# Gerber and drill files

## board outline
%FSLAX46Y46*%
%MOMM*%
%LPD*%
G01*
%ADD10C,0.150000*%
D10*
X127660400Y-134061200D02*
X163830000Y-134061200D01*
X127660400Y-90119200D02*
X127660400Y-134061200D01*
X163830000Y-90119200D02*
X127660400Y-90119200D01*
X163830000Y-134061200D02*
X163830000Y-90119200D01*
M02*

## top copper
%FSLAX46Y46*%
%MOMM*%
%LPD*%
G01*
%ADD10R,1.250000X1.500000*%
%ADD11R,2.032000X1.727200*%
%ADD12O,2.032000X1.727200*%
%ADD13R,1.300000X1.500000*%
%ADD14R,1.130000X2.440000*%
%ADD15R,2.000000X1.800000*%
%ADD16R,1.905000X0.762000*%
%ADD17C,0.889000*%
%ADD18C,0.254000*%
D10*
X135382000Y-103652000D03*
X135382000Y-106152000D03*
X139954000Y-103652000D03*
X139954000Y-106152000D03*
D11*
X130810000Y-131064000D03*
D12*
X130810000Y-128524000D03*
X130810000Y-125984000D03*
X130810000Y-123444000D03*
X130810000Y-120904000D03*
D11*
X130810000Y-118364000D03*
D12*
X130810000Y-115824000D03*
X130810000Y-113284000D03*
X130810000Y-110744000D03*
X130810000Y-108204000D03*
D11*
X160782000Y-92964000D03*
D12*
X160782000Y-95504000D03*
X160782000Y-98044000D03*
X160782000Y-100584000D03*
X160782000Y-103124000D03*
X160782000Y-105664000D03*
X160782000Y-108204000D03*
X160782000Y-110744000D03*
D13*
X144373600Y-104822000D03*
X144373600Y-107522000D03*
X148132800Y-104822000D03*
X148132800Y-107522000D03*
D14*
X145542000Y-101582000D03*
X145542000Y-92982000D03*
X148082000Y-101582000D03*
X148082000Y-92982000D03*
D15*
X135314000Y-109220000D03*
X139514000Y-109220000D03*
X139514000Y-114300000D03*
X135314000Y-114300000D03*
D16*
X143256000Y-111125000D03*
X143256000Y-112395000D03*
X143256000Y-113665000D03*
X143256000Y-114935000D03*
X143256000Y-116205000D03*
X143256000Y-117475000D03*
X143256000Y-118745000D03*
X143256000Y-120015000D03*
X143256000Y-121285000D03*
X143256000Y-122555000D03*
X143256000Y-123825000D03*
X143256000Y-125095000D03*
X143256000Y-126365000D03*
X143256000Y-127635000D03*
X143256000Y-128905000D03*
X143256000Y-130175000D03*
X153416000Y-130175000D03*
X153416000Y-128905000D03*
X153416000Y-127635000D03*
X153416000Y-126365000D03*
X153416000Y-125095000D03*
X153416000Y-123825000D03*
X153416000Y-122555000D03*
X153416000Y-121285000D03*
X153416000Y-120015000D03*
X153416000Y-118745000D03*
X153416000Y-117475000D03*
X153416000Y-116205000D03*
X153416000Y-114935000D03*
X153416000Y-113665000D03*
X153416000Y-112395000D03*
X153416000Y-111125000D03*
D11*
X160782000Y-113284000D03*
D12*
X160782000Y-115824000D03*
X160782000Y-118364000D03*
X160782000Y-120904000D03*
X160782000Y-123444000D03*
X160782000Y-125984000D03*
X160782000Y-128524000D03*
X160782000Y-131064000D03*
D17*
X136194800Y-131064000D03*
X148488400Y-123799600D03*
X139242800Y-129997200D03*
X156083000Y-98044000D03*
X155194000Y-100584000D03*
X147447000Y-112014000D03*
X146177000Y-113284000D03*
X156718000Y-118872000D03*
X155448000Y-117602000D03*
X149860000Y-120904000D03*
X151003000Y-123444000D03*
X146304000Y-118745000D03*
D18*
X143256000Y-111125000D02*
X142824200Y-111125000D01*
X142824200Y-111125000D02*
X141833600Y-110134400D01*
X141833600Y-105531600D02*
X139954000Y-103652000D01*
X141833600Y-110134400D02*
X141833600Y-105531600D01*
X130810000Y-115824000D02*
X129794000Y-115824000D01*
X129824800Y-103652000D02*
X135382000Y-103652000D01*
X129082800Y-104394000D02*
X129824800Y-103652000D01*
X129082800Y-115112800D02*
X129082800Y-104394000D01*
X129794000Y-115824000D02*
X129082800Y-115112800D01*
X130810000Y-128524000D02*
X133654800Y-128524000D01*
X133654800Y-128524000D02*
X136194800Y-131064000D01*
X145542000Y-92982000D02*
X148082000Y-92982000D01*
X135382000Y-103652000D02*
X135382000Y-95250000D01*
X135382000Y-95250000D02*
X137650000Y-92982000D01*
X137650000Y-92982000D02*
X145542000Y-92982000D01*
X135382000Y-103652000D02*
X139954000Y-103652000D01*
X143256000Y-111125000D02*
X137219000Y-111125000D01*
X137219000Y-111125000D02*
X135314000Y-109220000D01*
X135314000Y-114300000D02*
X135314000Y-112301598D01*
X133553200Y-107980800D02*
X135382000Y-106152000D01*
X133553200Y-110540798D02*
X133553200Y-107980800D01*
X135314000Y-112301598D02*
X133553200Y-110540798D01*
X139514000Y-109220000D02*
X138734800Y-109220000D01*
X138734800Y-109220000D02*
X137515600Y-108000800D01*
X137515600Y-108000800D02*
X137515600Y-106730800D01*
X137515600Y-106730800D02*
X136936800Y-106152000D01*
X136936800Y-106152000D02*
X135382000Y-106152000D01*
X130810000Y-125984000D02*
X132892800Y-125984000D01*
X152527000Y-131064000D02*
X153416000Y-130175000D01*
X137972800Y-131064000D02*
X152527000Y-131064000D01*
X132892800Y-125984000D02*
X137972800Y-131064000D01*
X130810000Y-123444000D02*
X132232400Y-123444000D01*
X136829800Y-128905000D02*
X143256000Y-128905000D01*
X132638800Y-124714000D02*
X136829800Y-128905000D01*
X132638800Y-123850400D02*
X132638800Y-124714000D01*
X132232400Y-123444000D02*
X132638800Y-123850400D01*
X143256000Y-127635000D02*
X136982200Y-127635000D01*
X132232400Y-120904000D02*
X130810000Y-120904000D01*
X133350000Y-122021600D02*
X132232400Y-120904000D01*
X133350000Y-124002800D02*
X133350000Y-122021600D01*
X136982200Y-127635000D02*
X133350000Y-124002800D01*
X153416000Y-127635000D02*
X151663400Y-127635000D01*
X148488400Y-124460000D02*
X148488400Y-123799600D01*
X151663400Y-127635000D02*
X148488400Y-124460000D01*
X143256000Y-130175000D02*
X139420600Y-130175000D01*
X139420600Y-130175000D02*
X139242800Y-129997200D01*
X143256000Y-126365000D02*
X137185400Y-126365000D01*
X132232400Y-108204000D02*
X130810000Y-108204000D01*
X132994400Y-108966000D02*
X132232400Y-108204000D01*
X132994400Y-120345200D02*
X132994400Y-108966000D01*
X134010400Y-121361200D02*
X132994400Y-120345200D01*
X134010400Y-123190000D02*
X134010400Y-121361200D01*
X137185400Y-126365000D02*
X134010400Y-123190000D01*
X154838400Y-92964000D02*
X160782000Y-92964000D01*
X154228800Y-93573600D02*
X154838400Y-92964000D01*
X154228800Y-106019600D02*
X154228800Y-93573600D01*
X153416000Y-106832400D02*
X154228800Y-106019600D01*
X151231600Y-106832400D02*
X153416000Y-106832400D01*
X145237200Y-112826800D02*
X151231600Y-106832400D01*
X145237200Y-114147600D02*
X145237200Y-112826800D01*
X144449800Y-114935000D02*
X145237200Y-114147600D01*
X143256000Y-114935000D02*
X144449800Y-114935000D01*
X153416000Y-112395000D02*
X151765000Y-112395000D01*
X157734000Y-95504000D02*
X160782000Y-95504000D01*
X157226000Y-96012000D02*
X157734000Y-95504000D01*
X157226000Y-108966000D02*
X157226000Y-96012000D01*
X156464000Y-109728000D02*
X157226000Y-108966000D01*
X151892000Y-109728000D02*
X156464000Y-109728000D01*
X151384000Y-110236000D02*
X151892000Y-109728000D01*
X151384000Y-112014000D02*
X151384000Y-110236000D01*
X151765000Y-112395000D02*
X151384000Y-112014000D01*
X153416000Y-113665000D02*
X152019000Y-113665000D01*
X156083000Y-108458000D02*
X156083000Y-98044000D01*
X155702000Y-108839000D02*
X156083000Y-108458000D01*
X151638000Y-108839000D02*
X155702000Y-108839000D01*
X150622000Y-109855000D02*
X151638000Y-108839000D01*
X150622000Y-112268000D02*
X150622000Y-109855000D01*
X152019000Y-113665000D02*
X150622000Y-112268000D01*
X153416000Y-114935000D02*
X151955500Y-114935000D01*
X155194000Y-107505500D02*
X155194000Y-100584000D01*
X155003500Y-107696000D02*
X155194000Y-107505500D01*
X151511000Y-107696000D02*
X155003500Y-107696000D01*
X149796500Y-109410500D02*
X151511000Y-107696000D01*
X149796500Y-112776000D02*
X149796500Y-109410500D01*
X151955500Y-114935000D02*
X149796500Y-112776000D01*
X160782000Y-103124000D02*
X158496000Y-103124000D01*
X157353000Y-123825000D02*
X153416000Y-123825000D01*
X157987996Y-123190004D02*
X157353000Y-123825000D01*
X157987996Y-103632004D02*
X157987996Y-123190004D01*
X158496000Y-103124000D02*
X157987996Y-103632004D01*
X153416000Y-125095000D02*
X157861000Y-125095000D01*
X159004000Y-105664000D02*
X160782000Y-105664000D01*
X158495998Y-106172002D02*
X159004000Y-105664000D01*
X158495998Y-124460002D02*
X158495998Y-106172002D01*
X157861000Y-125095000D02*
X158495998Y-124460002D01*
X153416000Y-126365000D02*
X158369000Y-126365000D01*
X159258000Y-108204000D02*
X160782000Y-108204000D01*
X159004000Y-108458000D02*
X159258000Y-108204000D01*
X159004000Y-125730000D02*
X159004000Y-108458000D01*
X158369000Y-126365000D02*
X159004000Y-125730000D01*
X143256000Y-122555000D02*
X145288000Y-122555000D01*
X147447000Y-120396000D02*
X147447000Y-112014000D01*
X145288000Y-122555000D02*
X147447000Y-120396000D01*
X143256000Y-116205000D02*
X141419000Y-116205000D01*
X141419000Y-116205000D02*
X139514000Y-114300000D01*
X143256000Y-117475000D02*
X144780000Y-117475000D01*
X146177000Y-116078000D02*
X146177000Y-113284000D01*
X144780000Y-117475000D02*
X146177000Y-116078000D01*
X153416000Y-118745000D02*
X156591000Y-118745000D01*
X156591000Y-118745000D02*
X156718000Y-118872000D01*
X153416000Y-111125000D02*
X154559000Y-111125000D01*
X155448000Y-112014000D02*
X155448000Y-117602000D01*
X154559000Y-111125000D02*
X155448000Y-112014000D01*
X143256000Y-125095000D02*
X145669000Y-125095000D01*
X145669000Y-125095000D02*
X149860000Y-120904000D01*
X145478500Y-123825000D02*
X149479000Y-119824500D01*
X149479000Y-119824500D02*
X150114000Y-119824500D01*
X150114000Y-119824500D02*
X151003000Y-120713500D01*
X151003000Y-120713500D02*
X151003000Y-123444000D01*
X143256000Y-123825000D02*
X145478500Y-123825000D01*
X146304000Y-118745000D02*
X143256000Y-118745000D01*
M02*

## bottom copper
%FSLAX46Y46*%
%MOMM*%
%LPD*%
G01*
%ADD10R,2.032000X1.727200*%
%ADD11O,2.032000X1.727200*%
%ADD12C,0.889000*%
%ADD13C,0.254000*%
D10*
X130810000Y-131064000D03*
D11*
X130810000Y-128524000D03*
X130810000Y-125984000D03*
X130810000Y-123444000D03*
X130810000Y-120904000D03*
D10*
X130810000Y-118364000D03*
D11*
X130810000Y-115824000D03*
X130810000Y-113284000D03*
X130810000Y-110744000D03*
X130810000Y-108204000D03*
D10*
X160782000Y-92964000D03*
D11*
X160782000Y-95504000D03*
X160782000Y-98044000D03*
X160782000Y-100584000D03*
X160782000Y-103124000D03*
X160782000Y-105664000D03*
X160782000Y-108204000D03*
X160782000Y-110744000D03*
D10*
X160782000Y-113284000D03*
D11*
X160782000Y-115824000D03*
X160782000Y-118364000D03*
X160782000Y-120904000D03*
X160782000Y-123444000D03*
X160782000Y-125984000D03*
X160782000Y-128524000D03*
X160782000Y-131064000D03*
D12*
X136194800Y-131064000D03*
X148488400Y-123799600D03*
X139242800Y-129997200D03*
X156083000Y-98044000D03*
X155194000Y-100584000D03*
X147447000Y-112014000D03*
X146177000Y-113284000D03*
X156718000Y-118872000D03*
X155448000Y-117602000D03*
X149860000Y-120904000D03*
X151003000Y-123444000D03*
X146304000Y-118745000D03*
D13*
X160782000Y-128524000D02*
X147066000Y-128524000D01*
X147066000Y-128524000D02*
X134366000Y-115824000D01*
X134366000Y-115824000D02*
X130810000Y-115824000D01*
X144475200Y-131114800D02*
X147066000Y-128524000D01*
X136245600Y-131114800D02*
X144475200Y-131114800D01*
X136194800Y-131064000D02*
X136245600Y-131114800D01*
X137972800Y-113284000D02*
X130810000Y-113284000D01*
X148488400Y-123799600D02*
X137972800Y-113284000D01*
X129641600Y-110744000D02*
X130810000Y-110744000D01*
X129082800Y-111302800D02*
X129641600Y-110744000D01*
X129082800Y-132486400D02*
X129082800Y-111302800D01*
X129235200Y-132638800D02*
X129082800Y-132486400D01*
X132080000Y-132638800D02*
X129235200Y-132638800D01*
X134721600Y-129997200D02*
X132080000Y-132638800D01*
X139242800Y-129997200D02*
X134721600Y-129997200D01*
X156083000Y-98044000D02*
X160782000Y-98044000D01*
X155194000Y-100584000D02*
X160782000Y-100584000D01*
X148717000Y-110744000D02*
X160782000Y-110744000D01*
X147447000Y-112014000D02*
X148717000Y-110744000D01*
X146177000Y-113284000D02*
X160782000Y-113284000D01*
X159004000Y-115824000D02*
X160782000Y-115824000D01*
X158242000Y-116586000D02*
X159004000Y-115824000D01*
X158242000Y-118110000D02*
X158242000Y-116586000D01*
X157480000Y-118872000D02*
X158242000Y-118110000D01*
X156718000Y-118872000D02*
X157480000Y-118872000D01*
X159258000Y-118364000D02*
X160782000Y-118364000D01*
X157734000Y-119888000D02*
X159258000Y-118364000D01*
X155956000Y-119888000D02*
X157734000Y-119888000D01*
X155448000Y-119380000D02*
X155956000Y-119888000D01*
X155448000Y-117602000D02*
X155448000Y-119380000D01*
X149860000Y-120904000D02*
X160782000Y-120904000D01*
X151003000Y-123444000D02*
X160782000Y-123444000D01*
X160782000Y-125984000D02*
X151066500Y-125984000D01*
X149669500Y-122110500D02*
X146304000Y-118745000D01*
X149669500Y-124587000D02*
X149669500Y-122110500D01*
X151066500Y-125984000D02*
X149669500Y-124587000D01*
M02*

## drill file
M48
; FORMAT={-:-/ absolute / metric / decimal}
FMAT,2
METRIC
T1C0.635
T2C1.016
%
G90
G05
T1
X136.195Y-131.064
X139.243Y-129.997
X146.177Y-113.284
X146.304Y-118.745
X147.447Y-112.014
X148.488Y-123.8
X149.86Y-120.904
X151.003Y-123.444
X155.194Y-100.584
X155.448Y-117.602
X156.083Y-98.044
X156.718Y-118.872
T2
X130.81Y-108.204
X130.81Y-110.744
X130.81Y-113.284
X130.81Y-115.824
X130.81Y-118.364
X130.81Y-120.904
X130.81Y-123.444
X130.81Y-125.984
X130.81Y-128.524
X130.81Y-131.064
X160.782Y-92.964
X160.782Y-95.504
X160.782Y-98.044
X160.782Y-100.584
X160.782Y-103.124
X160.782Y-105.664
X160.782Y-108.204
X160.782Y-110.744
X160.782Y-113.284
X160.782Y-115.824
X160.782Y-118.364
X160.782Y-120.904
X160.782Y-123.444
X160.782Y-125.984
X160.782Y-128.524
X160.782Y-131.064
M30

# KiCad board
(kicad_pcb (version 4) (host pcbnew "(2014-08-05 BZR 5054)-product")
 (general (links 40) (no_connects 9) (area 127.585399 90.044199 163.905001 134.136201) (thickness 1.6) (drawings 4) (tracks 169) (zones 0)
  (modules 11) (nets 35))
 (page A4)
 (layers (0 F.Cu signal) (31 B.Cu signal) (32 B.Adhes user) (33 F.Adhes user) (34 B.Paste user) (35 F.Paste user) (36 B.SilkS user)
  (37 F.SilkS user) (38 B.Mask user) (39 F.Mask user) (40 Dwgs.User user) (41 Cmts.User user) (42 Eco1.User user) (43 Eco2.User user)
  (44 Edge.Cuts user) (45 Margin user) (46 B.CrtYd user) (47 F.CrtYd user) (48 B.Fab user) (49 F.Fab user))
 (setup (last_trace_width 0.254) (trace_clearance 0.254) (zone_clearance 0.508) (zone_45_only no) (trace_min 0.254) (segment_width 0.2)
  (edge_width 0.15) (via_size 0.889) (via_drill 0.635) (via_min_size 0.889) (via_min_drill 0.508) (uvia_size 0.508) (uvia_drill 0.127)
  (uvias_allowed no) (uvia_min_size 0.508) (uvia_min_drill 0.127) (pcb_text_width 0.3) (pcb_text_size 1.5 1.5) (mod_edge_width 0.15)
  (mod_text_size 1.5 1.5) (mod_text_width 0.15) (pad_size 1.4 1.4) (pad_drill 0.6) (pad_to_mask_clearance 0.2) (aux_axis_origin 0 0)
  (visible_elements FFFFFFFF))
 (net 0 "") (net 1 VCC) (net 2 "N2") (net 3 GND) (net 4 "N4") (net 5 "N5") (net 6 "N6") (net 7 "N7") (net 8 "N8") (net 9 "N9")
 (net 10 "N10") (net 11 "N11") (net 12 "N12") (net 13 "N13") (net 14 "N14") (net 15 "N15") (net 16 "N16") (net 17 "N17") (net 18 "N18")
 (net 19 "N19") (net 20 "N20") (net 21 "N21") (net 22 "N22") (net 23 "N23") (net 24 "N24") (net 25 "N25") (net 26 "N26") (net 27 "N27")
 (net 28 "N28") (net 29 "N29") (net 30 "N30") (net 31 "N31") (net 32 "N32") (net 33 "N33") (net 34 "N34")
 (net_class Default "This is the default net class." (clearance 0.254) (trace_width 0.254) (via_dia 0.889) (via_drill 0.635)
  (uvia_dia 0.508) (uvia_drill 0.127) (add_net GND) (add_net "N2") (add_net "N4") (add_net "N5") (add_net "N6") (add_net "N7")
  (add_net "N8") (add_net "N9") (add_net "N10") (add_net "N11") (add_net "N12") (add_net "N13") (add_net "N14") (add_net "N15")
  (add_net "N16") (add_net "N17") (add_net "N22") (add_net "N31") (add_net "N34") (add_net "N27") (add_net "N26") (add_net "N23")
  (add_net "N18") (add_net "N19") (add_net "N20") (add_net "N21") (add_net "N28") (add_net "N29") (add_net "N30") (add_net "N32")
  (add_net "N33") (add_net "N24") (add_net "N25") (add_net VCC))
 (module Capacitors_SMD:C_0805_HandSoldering (layer F.Cu) (at 135.382 104.902 270)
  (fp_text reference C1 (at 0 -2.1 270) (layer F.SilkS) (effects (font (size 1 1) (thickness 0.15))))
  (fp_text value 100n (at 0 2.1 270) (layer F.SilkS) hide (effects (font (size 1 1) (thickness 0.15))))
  (pad 1 smd rect (at -1.25 0 270) (size 1.5 1.25) (layers F.Cu F.Paste F.Mask) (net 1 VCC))
  (pad 2 smd rect (at 1.25 0 270) (size 1.5 1.25) (layers F.Cu F.Paste F.Mask) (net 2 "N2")))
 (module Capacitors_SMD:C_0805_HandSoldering (layer F.Cu) (at 139.954 104.902 270) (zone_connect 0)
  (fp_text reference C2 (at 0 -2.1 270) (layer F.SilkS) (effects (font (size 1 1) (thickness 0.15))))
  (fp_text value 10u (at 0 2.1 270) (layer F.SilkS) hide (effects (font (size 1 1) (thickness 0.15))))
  (pad 1 smd rect (at -1.25 0 270) (size 1.5 1.25) (layers F.Cu F.Paste F.Mask) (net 1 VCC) (zone_connect 0))
  (pad 2 smd rect (at 1.25 0 270) (size 1.5 1.25) (layers F.Cu F.Paste F.Mask) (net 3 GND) (zone_connect 0)))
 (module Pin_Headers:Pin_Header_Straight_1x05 (layer F.Cu) (at 130.81 125.984 90)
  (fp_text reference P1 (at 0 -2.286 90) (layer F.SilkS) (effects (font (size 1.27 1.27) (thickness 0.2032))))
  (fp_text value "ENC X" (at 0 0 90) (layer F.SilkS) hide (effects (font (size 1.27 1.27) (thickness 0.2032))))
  (pad 1 thru_hole rect (at -5.08 0 90) (size 1.7272 2.032) (drill 1.016) (layers *.Cu *.Mask F.SilkS) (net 3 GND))
  (pad 2 thru_hole oval (at -2.54 0 90) (size 1.7272 2.032) (drill 1.016) (layers *.Cu *.Mask F.SilkS) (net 1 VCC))
  (pad 3 thru_hole oval (at 0 0 90) (size 1.7272 2.032) (drill 1.016) (layers *.Cu *.Mask F.SilkS) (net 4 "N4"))
  (pad 4 thru_hole oval (at 2.54 0 90) (size 1.7272 2.032) (drill 1.016) (layers *.Cu *.Mask F.SilkS) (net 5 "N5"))
  (pad 5 thru_hole oval (at 5.08 0 90) (size 1.7272 2.032) (drill 1.016) (layers *.Cu *.Mask F.SilkS) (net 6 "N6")))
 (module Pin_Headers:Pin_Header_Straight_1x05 (layer F.Cu) (at 130.81 113.284 90)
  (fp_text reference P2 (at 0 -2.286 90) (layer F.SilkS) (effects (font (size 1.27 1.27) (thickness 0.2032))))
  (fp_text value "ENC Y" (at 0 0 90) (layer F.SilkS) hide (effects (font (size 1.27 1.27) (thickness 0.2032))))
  (pad 1 thru_hole rect (at -5.08 0 90) (size 1.7272 2.032) (drill 1.016) (layers *.Cu *.Mask F.SilkS) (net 3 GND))
  (pad 2 thru_hole oval (at -2.54 0 90) (size 1.7272 2.032) (drill 1.016) (layers *.Cu *.Mask F.SilkS) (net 1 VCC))
  (pad 3 thru_hole oval (at 0 0 90) (size 1.7272 2.032) (drill 1.016) (layers *.Cu *.Mask F.SilkS) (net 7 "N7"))
  (pad 4 thru_hole oval (at 2.54 0 90) (size 1.7272 2.032) (drill 1.016) (layers *.Cu *.Mask F.SilkS) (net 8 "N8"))
  (pad 5 thru_hole oval (at 5.08 0 90) (size 1.7272 2.032) (drill 1.016) (layers *.Cu *.Mask F.SilkS) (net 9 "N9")))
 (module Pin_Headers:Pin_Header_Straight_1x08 (layer F.Cu) (at 160.782 101.854 270)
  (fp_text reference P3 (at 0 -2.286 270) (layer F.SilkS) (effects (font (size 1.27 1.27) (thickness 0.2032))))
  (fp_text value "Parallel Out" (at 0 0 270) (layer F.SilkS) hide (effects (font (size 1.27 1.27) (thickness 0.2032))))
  (pad 1 thru_hole rect (at -8.89 0 270) (size 1.7272 2.032) (drill 1.016) (layers *.Cu *.Mask F.SilkS) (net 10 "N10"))
  (pad 2 thru_hole oval (at -6.35 0 270) (size 1.7272 2.032) (drill 1.016) (layers *.Cu *.Mask F.SilkS) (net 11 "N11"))
  (pad 3 thru_hole oval (at -3.81 0 270) (size 1.7272 2.032) (drill 1.016) (layers *.Cu *.Mask F.SilkS) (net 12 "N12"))
  (pad 4 thru_hole oval (at -1.27 0 270) (size 1.7272 2.032) (drill 1.016) (layers *.Cu *.Mask F.SilkS) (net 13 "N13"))
  (pad 5 thru_hole oval (at 1.27 0 270) (size 1.7272 2.032) (drill 1.016) (layers *.Cu *.Mask F.SilkS) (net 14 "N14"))
  (pad 6 thru_hole oval (at 3.81 0 270) (size 1.7272 2.032) (drill 1.016) (layers *.Cu *.Mask F.SilkS) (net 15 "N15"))
  (pad 7 thru_hole oval (at 6.35 0 270) (size 1.7272 2.032) (drill 1.016) (layers *.Cu *.Mask F.SilkS) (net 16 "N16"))
  (pad 8 thru_hole oval (at 8.89 0 270) (size 1.7272 2.032) (drill 1.016) (layers *.Cu *.Mask F.SilkS) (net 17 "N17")))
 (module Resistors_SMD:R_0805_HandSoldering (layer F.Cu) (at 144.3736 106.172 270)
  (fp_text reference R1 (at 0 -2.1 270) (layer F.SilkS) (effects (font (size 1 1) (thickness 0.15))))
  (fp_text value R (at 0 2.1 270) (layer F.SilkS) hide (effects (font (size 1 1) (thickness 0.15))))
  (pad 1 smd rect (at -1.35 0 270) (size 1.5 1.3) (layers F.Cu F.Paste F.Mask) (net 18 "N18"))
  (pad 2 smd rect (at 1.35 0 270) (size 1.5 1.3) (layers F.Cu F.Paste F.Mask) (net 3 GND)))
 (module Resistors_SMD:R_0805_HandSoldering (layer F.Cu) (at 148.1328 106.172 270)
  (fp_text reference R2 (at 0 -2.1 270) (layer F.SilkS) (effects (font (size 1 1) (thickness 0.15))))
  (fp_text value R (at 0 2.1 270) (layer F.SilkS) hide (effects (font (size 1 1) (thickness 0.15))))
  (pad 1 smd rect (at -1.35 0 270) (size 1.5 1.3) (layers F.Cu F.Paste F.Mask) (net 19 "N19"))
  (pad 2 smd rect (at 1.35 0 270) (size 1.5 1.3) (layers F.Cu F.Paste F.Mask) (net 3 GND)))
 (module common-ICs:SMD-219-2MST (layer F.Cu) (at 146.812 97.282)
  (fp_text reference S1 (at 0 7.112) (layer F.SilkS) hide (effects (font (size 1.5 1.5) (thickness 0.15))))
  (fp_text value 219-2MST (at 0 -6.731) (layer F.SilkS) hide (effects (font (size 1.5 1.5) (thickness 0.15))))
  (pad 3 smd rect (at -1.27 4.3) (size 1.13 2.44) (layers F.Cu F.Paste F.Mask) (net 18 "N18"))
  (pad 2 smd rect (at -1.27 -4.3) (size 1.13 2.44) (layers F.Cu F.Paste F.Mask) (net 1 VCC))
  (pad 4 smd rect (at 1.27 4.3) (size 1.13 2.44) (layers F.Cu F.Paste F.Mask) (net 19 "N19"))
  (pad 1 smd rect (at 1.27 -4.3) (size 1.13 2.44) (layers F.Cu F.Paste F.Mask) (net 1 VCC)))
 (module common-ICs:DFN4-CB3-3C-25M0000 (layer F.Cu) (at 137.414 111.76 270)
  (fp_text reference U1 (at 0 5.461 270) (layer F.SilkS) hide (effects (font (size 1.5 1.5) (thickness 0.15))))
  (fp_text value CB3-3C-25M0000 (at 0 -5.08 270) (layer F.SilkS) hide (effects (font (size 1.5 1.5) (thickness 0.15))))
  (pad 1 smd rect (at -2.54 2.1 270) (size 1.8 2) (layers F.Cu F.Paste F.Mask) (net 1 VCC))
  (pad 2 smd rect (at -2.54 -2.1 270) (size 1.8 2) (layers F.Cu F.Paste F.Mask) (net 2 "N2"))
  (pad 3 smd rect (at 2.54 -2.1 270) (size 1.8 2) (layers F.Cu F.Paste F.Mask) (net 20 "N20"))
  (pad 2 smd rect (at 2.54 2.1 270) (size 1.8 2) (layers F.Cu F.Paste F.Mask) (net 2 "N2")))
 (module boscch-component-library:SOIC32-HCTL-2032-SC (layer F.Cu) (at 148.336 120.65)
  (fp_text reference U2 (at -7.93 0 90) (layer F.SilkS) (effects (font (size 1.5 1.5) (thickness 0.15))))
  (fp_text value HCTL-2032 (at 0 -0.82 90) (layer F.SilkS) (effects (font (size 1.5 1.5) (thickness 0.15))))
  (pad 1 smd rect (at -5.08 -9.525) (size 1.905 0.762) (layers F.Cu F.Paste F.Mask) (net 1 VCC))
  (pad 2 smd rect (at -5.08 -8.255) (size 1.905 0.762) (layers F.Cu F.Paste F.Mask) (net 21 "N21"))
  (pad 3 smd rect (at -5.08 -6.985) (size 1.905 0.762) (layers F.Cu F.Paste F.Mask) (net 18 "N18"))
  (pad 4 smd rect (at -5.08 -5.715) (size 1.905 0.762) (layers F.Cu F.Paste F.Mask) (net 10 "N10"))
  (pad 5 smd rect (at -5.08 -4.445) (size 1.905 0.762) (layers F.Cu F.Paste F.Mask) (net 20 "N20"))
  (pad 6 smd rect (at -5.08 -3.175) (size 1.905 0.762) (layers F.Cu F.Paste F.Mask) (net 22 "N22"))
  (pad 7 smd rect (at -5.08 -1.905) (size 1.905 0.762) (layers F.Cu F.Paste F.Mask) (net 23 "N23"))
  (pad 8 smd rect (at -5.08 -0.635) (size 1.905 0.762) (layers F.Cu F.Paste F.Mask) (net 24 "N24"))
  (pad 9 smd rect (at -5.08 0.635) (size 1.905 0.762) (layers F.Cu F.Paste F.Mask) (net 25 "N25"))
  (pad 10 smd rect (at -5.08 1.905) (size 1.905 0.762) (layers F.Cu F.Paste F.Mask) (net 17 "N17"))
  (pad 11 smd rect (at -5.08 3.175) (size 1.905 0.762) (layers F.Cu F.Paste F.Mask) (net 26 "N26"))
  (pad 12 smd rect (at -5.08 4.445) (size 1.905 0.762) (layers F.Cu F.Paste F.Mask) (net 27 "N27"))
  (pad 13 smd rect (at -5.08 5.715) (size 1.905 0.762) (layers F.Cu F.Paste F.Mask) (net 9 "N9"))
  (pad 14 smd rect (at -5.08 6.985) (size 1.905 0.762) (layers F.Cu F.Paste F.Mask) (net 6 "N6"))
  (pad 15 smd rect (at -5.08 8.255) (size 1.905 0.762) (layers F.Cu F.Paste F.Mask) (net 5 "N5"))
  (pad 16 smd rect (at -5.08 9.525) (size 1.905 0.762) (layers F.Cu F.Paste F.Mask) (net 8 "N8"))
  (pad 17 smd rect (at 5.08 9.525) (size 1.905 0.762) (layers F.Cu F.Paste F.Mask) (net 4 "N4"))
  (pad 18 smd rect (at 5.08 8.255) (size 1.905 0.762) (layers F.Cu F.Paste F.Mask) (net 3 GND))
  (pad 19 smd rect (at 5.08 6.985) (size 1.905 0.762) (layers F.Cu F.Paste F.Mask) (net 7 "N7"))
  (pad 20 smd rect (at 5.08 5.715) (size 1.905 0.762) (layers F.Cu F.Paste F.Mask) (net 16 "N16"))
  (pad 21 smd rect (at 5.08 4.445) (size 1.905 0.762) (layers F.Cu F.Paste F.Mask) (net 15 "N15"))
  (pad 22 smd rect (at 5.08 3.175) (size 1.905 0.762) (layers F.Cu F.Paste F.Mask) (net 14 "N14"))
  (pad 23 smd rect (at 5.08 1.905) (size 1.905 0.762) (layers F.Cu F.Paste F.Mask) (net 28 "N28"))
  (pad 24 smd rect (at 5.08 0.635) (size 1.905 0.762) (layers F.Cu F.Paste F.Mask) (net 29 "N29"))
  (pad 25 smd rect (at 5.08 -0.635) (size 1.905 0.762) (layers F.Cu F.Paste F.Mask) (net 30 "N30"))
  (pad 26 smd rect (at 5.08 -1.905) (size 1.905 0.762) (layers F.Cu F.Paste F.Mask) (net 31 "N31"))
  (pad 27 smd rect (at 5.08 -3.175) (size 1.905 0.762) (layers F.Cu F.Paste F.Mask) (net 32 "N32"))
  (pad 28 smd rect (at 5.08 -4.445) (size 1.905 0.762) (layers F.Cu F.Paste F.Mask) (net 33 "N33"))
  (pad 29 smd rect (at 5.08 -5.715) (size 1.905 0.762) (layers F.Cu F.Paste F.Mask) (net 13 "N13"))
  (pad 30 smd rect (at 5.08 -6.985) (size 1.905 0.762) (layers F.Cu F.Paste F.Mask) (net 12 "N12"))
  (pad 31 smd rect (at 5.08 -8.255) (size 1.905 0.762) (layers F.Cu F.Paste F.Mask) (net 11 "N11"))
  (pad 32 smd rect (at 5.08 -9.525) (size 1.905 0.762) (layers F.Cu F.Paste F.Mask) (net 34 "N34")))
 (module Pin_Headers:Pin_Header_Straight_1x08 (layer F.Cu) (at 160.782 122.174 270)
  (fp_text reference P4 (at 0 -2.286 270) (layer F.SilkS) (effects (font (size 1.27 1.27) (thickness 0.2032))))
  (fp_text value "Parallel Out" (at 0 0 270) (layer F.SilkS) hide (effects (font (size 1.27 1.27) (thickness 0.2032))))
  (pad 1 thru_hole rect (at -8.89 0 270) (size 1.7272 2.032) (drill 1.016) (layers *.Cu *.Mask F.SilkS) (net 22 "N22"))
  (pad 2 thru_hole oval (at -6.35 0 270) (size 1.7272 2.032) (drill 1.016) (layers *.Cu *.Mask F.SilkS) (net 31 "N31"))
  (pad 3 thru_hole oval (at -3.81 0 270) (size 1.7272 2.032) (drill 1.016) (layers *.Cu *.Mask F.SilkS) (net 34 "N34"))
  (pad 4 thru_hole oval (at -1.27 0 270) (size 1.7272 2.032) (drill 1.016) (layers *.Cu *.Mask F.SilkS) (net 27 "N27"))
  (pad 5 thru_hole oval (at 1.27 0 270) (size 1.7272 2.032) (drill 1.016) (layers *.Cu *.Mask F.SilkS) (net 26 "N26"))
  (pad 6 thru_hole oval (at 3.81 0 270) (size 1.7272 2.032) (drill 1.016) (layers *.Cu *.Mask F.SilkS) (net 23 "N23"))
  (pad 7 thru_hole oval (at 6.35 0 270) (size 1.7272 2.032) (drill 1.016) (layers *.Cu *.Mask F.SilkS) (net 1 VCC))
  (pad 8 thru_hole oval (at 8.89 0 270) (size 1.7272 2.032) (drill 1.016) (layers *.Cu *.Mask F.SilkS) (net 3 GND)))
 (gr_line (start 127.6604 134.0612) (end 163.83 134.0612) (angle 90) (layer Edge.Cuts) (width 0.15))
 (gr_line (start 127.6604 90.1192) (end 127.6604 134.0612) (angle 90) (layer Edge.Cuts) (width 0.15))
 (gr_line (start 163.83 90.1192) (end 127.6604 90.1192) (angle 90) (layer Edge.Cuts) (width 0.15))
 (gr_line (start 163.83 134.0612) (end 163.83 90.1192) (angle 90) (layer Edge.Cuts) (width 0.15))
 (segment (start 143.256 111.125) (end 142.8242 111.125) (width 0.254) (layer F.Cu) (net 1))
 (segment (start 142.8242 111.125) (end 141.8336 110.1344) (width 0.254) (layer F.Cu) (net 1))
 (segment (start 141.8336 105.5316) (end 139.954 103.652) (width 0.254) (layer F.Cu) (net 1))
 (segment (start 141.8336 110.1344) (end 141.8336 105.5316) (width 0.254) (layer F.Cu) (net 1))
 (segment (start 130.81 115.824) (end 129.794 115.824) (width 0.254) (layer F.Cu) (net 1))
 (segment (start 129.8248 103.652) (end 135.382 103.652) (width 0.254) (layer F.Cu) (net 1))
 (segment (start 129.0828 104.394) (end 129.8248 103.652) (width 0.254) (layer F.Cu) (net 1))
 (segment (start 129.0828 115.1128) (end 129.0828 104.394) (width 0.254) (layer F.Cu) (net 1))
 (segment (start 129.794 115.824) (end 129.0828 115.1128) (width 0.254) (layer F.Cu) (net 1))
 (segment (start 160.782 128.524) (end 147.066 128.524) (width 0.254) (layer B.Cu) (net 1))
 (segment (start 147.066 128.524) (end 134.366 115.824) (width 0.254) (layer B.Cu) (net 1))
 (segment (start 134.366 115.824) (end 130.81 115.824) (width 0.254) (layer B.Cu) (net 1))
 (segment (start 130.81 128.524) (end 133.6548 128.524) (width 0.254) (layer F.Cu) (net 1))
 (segment (start 144.4752 131.1148) (end 147.066 128.524) (width 0.254) (layer B.Cu) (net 1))
 (segment (start 136.2456 131.1148) (end 144.4752 131.1148) (width 0.254) (layer B.Cu) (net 1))
 (segment (start 136.1948 131.064) (end 136.2456 131.1148) (width 0.254) (layer B.Cu) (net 1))
 (via (at 136.1948 131.064) (size 0.889) (layers F.Cu B.Cu) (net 1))
 (segment (start 133.6548 128.524) (end 136.1948 131.064) (width 0.254) (layer F.Cu) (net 1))
 (segment (start 145.542 92.982) (end 148.082 92.982) (width 0.254) (layer F.Cu) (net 1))
 (segment (start 135.382 103.652) (end 135.382 95.25) (width 0.254) (layer F.Cu) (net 1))
 (segment (start 135.382 95.25) (end 137.65 92.982) (width 0.254) (layer F.Cu) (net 1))
 (segment (start 137.65 92.982) (end 145.542 92.982) (width 0.254) (layer F.Cu) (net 1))
 (segment (start 135.382 103.652) (end 139.954 103.652) (width 0.254) (layer F.Cu) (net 1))
 (segment (start 143.256 111.125) (end 137.219 111.125) (width 0.254) (layer F.Cu) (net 1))
 (segment (start 137.219 111.125) (end 135.314 109.22) (width 0.254) (layer F.Cu) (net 1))
 (segment (start 135.314 114.3) (end 135.314 112.301598) (width 0.254) (layer F.Cu) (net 2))
 (segment (start 133.5532 107.9808) (end 135.382 106.152) (width 0.254) (layer F.Cu) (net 2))
 (segment (start 133.5532 110.540798) (end 133.5532 107.9808) (width 0.254) (layer F.Cu) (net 2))
 (segment (start 135.314 112.301598) (end 133.5532 110.540798) (width 0.254) (layer F.Cu) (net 2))
 (segment (start 139.514 109.22) (end 138.7348 109.22) (width 0.254) (layer F.Cu) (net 2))
 (segment (start 138.7348 109.22) (end 137.5156 108.0008) (width 0.254) (layer F.Cu) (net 2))
 (segment (start 137.5156 108.0008) (end 137.5156 106.7308) (width 0.254) (layer F.Cu) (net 2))
 (segment (start 137.5156 106.7308) (end 136.9368 106.152) (width 0.254) (layer F.Cu) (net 2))
 (segment (start 136.9368 106.152) (end 135.382 106.152) (width 0.254) (layer F.Cu) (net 2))
 (segment (start 130.81 125.984) (end 132.8928 125.984) (width 0.254) (layer F.Cu) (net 4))
 (segment (start 152.527 131.064) (end 153.416 130.175) (width 0.254) (layer F.Cu) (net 4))
 (segment (start 137.9728 131.064) (end 152.527 131.064) (width 0.254) (layer F.Cu) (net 4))
 (segment (start 132.8928 125.984) (end 137.9728 131.064) (width 0.254) (layer F.Cu) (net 4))
 (segment (start 130.81 123.444) (end 132.2324 123.444) (width 0.254) (layer F.Cu) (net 5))
 (segment (start 136.8298 128.905) (end 143.256 128.905) (width 0.254) (layer F.Cu) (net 5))
 (segment (start 132.6388 124.714) (end 136.8298 128.905) (width 0.254) (layer F.Cu) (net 5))
 (segment (start 132.6388 123.8504) (end 132.6388 124.714) (width 0.254) (layer F.Cu) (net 5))
 (segment (start 132.2324 123.444) (end 132.6388 123.8504) (width 0.254) (layer F.Cu) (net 5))
 (segment (start 143.256 127.635) (end 136.9822 127.635) (width 0.254) (layer F.Cu) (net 6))
 (segment (start 132.2324 120.904) (end 130.81 120.904) (width 0.254) (layer F.Cu) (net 6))
 (segment (start 133.35 122.0216) (end 132.2324 120.904) (width 0.254) (layer F.Cu) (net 6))
 (segment (start 133.35 124.0028) (end 133.35 122.0216) (width 0.254) (layer F.Cu) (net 6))
 (segment (start 136.9822 127.635) (end 133.35 124.0028) (width 0.254) (layer F.Cu) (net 6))
 (segment (start 153.416 127.635) (end 151.6634 127.635) (width 0.254) (layer F.Cu) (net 7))
 (segment (start 137.9728 113.284) (end 130.81 113.284) (width 0.254) (layer B.Cu) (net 7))
 (segment (start 148.4884 123.7996) (end 137.9728 113.284) (width 0.254) (layer B.Cu) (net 7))
 (via (at 148.4884 123.7996) (size 0.889) (layers F.Cu B.Cu) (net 7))
 (segment (start 148.4884 124.46) (end 148.4884 123.7996) (width 0.254) (layer F.Cu) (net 7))
 (segment (start 151.6634 127.635) (end 148.4884 124.46) (width 0.254) (layer F.Cu) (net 7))
 (segment (start 143.256 130.175) (end 139.4206 130.175) (width 0.254) (layer F.Cu) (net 8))
 (segment (start 129.6416 110.744) (end 130.81 110.744) (width 0.254) (layer B.Cu) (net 8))
 (segment (start 129.0828 111.3028) (end 129.6416 110.744) (width 0.254) (layer B.Cu) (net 8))
 (segment (start 129.0828 132.4864) (end 129.0828 111.3028) (width 0.254) (layer B.Cu) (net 8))
 (segment (start 129.2352 132.6388) (end 129.0828 132.4864) (width 0.254) (layer B.Cu) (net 8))
 (segment (start 132.08 132.6388) (end 129.2352 132.6388) (width 0.254) (layer B.Cu) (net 8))
 (segment (start 134.7216 129.9972) (end 132.08 132.6388) (width 0.254) (layer B.Cu) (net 8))
 (segment (start 139.2428 129.9972) (end 134.7216 129.9972) (width 0.254) (layer B.Cu) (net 8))
 (via (at 139.2428 129.9972) (size 0.889) (layers F.Cu B.Cu) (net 8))
 (segment (start 139.4206 130.175) (end 139.2428 129.9972) (width 0.254) (layer F.Cu) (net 8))
 (segment (start 143.256 126.365) (end 137.1854 126.365) (width 0.254) (layer F.Cu) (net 9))
 (segment (start 132.2324 108.204) (end 130.81 108.204) (width 0.254) (layer F.Cu) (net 9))
 (segment (start 132.9944 108.966) (end 132.2324 108.204) (width 0.254) (layer F.Cu) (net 9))
 (segment (start 132.9944 120.3452) (end 132.9944 108.966) (width 0.254) (layer F.Cu) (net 9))
 (segment (start 134.0104 121.3612) (end 132.9944 120.3452) (width 0.254) (layer F.Cu) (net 9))
 (segment (start 134.0104 123.19) (end 134.0104 121.3612) (width 0.254) (layer F.Cu) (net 9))
 (segment (start 137.1854 126.365) (end 134.0104 123.19) (width 0.254) (layer F.Cu) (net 9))
 (segment (start 154.8384 92.964) (end 160.782 92.964) (width 0.254) (layer F.Cu) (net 10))
 (segment (start 154.2288 93.5736) (end 154.8384 92.964) (width 0.254) (layer F.Cu) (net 10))
 (segment (start 154.2288 106.0196) (end 154.2288 93.5736) (width 0.254) (layer F.Cu) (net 10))
 (segment (start 153.416 106.8324) (end 154.2288 106.0196) (width 0.254) (layer F.Cu) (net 10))
 (segment (start 151.2316 106.8324) (end 153.416 106.8324) (width 0.254) (layer F.Cu) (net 10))
 (segment (start 145.2372 112.8268) (end 151.2316 106.8324) (width 0.254) (layer F.Cu) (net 10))
 (segment (start 145.2372 114.1476) (end 145.2372 112.8268) (width 0.254) (layer F.Cu) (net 10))
 (segment (start 144.4498 114.935) (end 145.2372 114.1476) (width 0.254) (layer F.Cu) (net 10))
 (segment (start 143.256 114.935) (end 144.4498 114.935) (width 0.254) (layer F.Cu) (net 10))
 (segment (start 153.416 112.395) (end 151.765 112.395) (width 0.254) (layer F.Cu) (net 11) (status 10))
 (segment (start 157.734 95.504) (end 160.782 95.504) (width 0.254) (layer F.Cu) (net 11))
 (segment (start 157.226 96.012) (end 157.734 95.504) (width 0.254) (layer F.Cu) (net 11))
 (segment (start 157.226 108.966) (end 157.226 96.012) (width 0.254) (layer F.Cu) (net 11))
 (segment (start 156.464 109.728) (end 157.226 108.966) (width 0.254) (layer F.Cu) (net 11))
 (segment (start 151.892 109.728) (end 156.464 109.728) (width 0.254) (layer F.Cu) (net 11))
 (segment (start 151.384 110.236) (end 151.892 109.728) (width 0.254) (layer F.Cu) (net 11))
 (segment (start 151.384 112.014) (end 151.384 110.236) (width 0.254) (layer F.Cu) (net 11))
 (segment (start 151.765 112.395) (end 151.384 112.014) (width 0.254) (layer F.Cu) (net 11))
 (segment (start 153.416 113.665) (end 152.019 113.665) (width 0.254) (layer F.Cu) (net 12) (status 10))
 (segment (start 156.083 98.044) (end 160.782 98.044) (width 0.254) (layer B.Cu) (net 12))
 (via (at 156.083 98.044) (size 0.889) (layers F.Cu B.Cu) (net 12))
 (segment (start 156.083 108.458) (end 156.083 98.044) (width 0.254) (layer F.Cu) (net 12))
 (segment (start 155.702 108.839) (end 156.083 108.458) (width 0.254) (layer F.Cu) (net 12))
 (segment (start 151.638 108.839) (end 155.702 108.839) (width 0.254) (layer F.Cu) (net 12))
 (segment (start 150.622 109.855) (end 151.638 108.839) (width 0.254) (layer F.Cu) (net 12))
 (segment (start 150.622 112.268) (end 150.622 109.855) (width 0.254) (layer F.Cu) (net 12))
 (segment (start 152.019 113.665) (end 150.622 112.268) (width 0.254) (layer F.Cu) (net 12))
 (segment (start 153.416 114.935) (end 151.9555 114.935) (width 0.254) (layer F.Cu) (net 13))
 (segment (start 155.194 100.584) (end 160.782 100.584) (width 0.254) (layer B.Cu) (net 13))
 (via (at 155.194 100.584) (size 0.889) (layers F.Cu B.Cu) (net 13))
 (segment (start 155.194 107.5055) (end 155.194 100.584) (width 0.254) (layer F.Cu) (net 13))
 (segment (start 155.0035 107.696) (end 155.194 107.5055) (width 0.254) (layer F.Cu) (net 13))
 (segment (start 151.511 107.696) (end 155.0035 107.696) (width 0.254) (layer F.Cu) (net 13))
 (segment (start 149.7965 109.4105) (end 151.511 107.696) (width 0.254) (layer F.Cu) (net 13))
 (segment (start 149.7965 112.776) (end 149.7965 109.4105) (width 0.254) (layer F.Cu) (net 13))
 (segment (start 151.9555 114.935) (end 149.7965 112.776) (width 0.254) (layer F.Cu) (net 13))
 (segment (start 160.782 103.124) (end 158.496 103.124) (width 0.254) (layer F.Cu) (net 14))
 (segment (start 157.353 123.825) (end 153.416 123.825) (width 0.254) (layer F.Cu) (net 14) (status 20))
 (segment (start 157.987996 123.190004) (end 157.353 123.825) (width 0.254) (layer F.Cu) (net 14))
 (segment (start 157.987996 103.632004) (end 157.987996 123.190004) (width 0.254) (layer F.Cu) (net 14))
 (segment (start 158.496 103.124) (end 157.987996 103.632004) (width 0.254) (layer F.Cu) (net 14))
 (segment (start 153.416 125.095) (end 157.861 125.095) (width 0.254) (layer F.Cu) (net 15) (status 10))
 (segment (start 159.004 105.664) (end 160.782 105.664) (width 0.254) (layer F.Cu) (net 15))
 (segment (start 158.495998 106.172002) (end 159.004 105.664) (width 0.254) (layer F.Cu) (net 15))
 (segment (start 158.495998 124.460002) (end 158.495998 106.172002) (width 0.254) (layer F.Cu) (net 15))
 (segment (start 157.861 125.095) (end 158.495998 124.460002) (width 0.254) (layer F.Cu) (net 15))
 (segment (start 153.416 126.365) (end 158.369 126.365) (width 0.254) (layer F.Cu) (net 16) (status 10))
 (segment (start 159.258 108.204) (end 160.782 108.204) (width 0.254) (layer F.Cu) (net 16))
 (segment (start 159.004 108.458) (end 159.258 108.204) (width 0.254) (layer F.Cu) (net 16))
 (segment (start 159.004 125.73) (end 159.004 108.458) (width 0.254) (layer F.Cu) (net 16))
 (segment (start 158.369 126.365) (end 159.004 125.73) (width 0.254) (layer F.Cu) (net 16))
 (segment (start 143.256 122.555) (end 145.288 122.555) (width 0.254) (layer F.Cu) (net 17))
 (segment (start 148.717 110.744) (end 160.782 110.744) (width 0.254) (layer B.Cu) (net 17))
 (segment (start 147.447 112.014) (end 148.717 110.744) (width 0.254) (layer B.Cu) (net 17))
 (via (at 147.447 112.014) (size 0.889) (layers F.Cu B.Cu) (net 17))
 (segment (start 147.447 120.396) (end 147.447 112.014) (width 0.254) (layer F.Cu) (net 17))
 (segment (start 145.288 122.555) (end 147.447 120.396) (width 0.254) (layer F.Cu) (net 17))
 (segment (start 143.256 116.205) (end 141.419 116.205) (width 0.254) (layer F.Cu) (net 20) (status 10))
 (segment (start 141.419 116.205) (end 139.514 114.3) (width 0.254) (layer F.Cu) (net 20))
 (segment (start 143.256 117.475) (end 144.78 117.475) (width 0.254) (layer F.Cu) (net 22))
 (segment (start 146.177 113.284) (end 160.782 113.284) (width 0.254) (layer B.Cu) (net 22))
 (via (at 146.177 113.284) (size 0.889) (layers F.Cu B.Cu) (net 22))
 (segment (start 146.177 116.078) (end 146.177 113.284) (width 0.254) (layer F.Cu) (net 22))
 (segment (start 144.78 117.475) (end 146.177 116.078) (width 0.254) (layer F.Cu) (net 22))
 (segment (start 153.416 118.745) (end 156.591 118.745) (width 0.254) (layer F.Cu) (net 31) (status 10))
 (segment (start 159.004 115.824) (end 160.782 115.824) (width 0.254) (layer B.Cu) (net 31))
 (segment (start 158.242 116.586) (end 159.004 115.824) (width 0.254) (layer B.Cu) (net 31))
 (segment (start 158.242 118.11) (end 158.242 116.586) (width 0.254) (layer B.Cu) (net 31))
 (segment (start 157.48 118.872) (end 158.242 118.11) (width 0.254) (layer B.Cu) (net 31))
 (segment (start 156.718 118.872) (end 157.48 118.872) (width 0.254) (layer B.Cu) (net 31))
 (via (at 156.718 118.872) (size 0.889) (layers F.Cu B.Cu) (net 31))
 (segment (start 156.591 118.745) (end 156.718 118.872) (width 0.254) (layer F.Cu) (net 31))
 (segment (start 153.416 111.125) (end 154.559 111.125) (width 0.254) (layer F.Cu) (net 34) (status 10))
 (segment (start 159.258 118.364) (end 160.782 118.364) (width 0.254) (layer B.Cu) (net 34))
 (segment (start 157.734 119.888) (end 159.258 118.364) (width 0.254) (layer B.Cu) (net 34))
 (segment (start 155.956 119.888) (end 157.734 119.888) (width 0.254) (layer B.Cu) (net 34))
 (segment (start 155.448 119.38) (end 155.956 119.888) (width 0.254) (layer B.Cu) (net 34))
 (segment (start 155.448 117.602) (end 155.448 119.38) (width 0.254) (layer B.Cu) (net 34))
 (via (at 155.448 117.602) (size 0.889) (layers F.Cu B.Cu) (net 34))
 (segment (start 155.448 112.014) (end 155.448 117.602) (width 0.254) (layer F.Cu) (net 34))
 (segment (start 154.559 111.125) (end 155.448 112.014) (width 0.254) (layer F.Cu) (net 34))
 (segment (start 143.256 125.095) (end 145.669 125.095) (width 0.254) (layer F.Cu) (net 27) (status 10))
 (segment (start 149.86 120.904) (end 160.782 120.904) (width 0.254) (layer B.Cu) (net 27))
 (via (at 149.86 120.904) (size 0.889) (layers F.Cu B.Cu) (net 27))
 (segment (start 145.669 125.095) (end 149.86 120.904) (width 0.254) (layer F.Cu) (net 27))
 (via (at 151.003 123.444) (size 0.889) (layers F.Cu B.Cu) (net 26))
 (segment (start 145.4785 123.825) (end 149.479 119.8245) (width 0.254) (layer F.Cu) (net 26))
 (segment (start 149.479 119.8245) (end 150.114 119.8245) (width 0.254) (layer F.Cu) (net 26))
 (segment (start 150.114 119.8245) (end 151.003 120.7135) (width 0.254) (layer F.Cu) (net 26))
 (segment (start 151.003 120.7135) (end 151.003 123.444) (width 0.254) (layer F.Cu) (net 26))
 (segment (start 143.256 123.825) (end 145.4785 123.825) (width 0.254) (layer F.Cu) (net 26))
 (segment (start 151.003 123.444) (end 160.782 123.444) (width 0.254) (layer B.Cu) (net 26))
 (segment (start 160.782 125.984) (end 151.0665 125.984) (width 0.254) (layer B.Cu) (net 23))
 (segment (start 146.304 118.745) (end 143.256 118.745) (width 0.254) (layer F.Cu) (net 23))
 (via (at 146.304 118.745) (size 0.889) (layers F.Cu B.Cu) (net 23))
 (segment (start 149.6695 122.1105) (end 146.304 118.745) (width 0.254) (layer B.Cu) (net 23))
 (segment (start 149.6695 124.587) (end 149.6695 122.1105) (width 0.254) (layer B.Cu) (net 23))
 (segment (start 151.0665 125.984) (end 149.6695 124.587) (width 0.254) (layer B.Cu) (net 23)))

